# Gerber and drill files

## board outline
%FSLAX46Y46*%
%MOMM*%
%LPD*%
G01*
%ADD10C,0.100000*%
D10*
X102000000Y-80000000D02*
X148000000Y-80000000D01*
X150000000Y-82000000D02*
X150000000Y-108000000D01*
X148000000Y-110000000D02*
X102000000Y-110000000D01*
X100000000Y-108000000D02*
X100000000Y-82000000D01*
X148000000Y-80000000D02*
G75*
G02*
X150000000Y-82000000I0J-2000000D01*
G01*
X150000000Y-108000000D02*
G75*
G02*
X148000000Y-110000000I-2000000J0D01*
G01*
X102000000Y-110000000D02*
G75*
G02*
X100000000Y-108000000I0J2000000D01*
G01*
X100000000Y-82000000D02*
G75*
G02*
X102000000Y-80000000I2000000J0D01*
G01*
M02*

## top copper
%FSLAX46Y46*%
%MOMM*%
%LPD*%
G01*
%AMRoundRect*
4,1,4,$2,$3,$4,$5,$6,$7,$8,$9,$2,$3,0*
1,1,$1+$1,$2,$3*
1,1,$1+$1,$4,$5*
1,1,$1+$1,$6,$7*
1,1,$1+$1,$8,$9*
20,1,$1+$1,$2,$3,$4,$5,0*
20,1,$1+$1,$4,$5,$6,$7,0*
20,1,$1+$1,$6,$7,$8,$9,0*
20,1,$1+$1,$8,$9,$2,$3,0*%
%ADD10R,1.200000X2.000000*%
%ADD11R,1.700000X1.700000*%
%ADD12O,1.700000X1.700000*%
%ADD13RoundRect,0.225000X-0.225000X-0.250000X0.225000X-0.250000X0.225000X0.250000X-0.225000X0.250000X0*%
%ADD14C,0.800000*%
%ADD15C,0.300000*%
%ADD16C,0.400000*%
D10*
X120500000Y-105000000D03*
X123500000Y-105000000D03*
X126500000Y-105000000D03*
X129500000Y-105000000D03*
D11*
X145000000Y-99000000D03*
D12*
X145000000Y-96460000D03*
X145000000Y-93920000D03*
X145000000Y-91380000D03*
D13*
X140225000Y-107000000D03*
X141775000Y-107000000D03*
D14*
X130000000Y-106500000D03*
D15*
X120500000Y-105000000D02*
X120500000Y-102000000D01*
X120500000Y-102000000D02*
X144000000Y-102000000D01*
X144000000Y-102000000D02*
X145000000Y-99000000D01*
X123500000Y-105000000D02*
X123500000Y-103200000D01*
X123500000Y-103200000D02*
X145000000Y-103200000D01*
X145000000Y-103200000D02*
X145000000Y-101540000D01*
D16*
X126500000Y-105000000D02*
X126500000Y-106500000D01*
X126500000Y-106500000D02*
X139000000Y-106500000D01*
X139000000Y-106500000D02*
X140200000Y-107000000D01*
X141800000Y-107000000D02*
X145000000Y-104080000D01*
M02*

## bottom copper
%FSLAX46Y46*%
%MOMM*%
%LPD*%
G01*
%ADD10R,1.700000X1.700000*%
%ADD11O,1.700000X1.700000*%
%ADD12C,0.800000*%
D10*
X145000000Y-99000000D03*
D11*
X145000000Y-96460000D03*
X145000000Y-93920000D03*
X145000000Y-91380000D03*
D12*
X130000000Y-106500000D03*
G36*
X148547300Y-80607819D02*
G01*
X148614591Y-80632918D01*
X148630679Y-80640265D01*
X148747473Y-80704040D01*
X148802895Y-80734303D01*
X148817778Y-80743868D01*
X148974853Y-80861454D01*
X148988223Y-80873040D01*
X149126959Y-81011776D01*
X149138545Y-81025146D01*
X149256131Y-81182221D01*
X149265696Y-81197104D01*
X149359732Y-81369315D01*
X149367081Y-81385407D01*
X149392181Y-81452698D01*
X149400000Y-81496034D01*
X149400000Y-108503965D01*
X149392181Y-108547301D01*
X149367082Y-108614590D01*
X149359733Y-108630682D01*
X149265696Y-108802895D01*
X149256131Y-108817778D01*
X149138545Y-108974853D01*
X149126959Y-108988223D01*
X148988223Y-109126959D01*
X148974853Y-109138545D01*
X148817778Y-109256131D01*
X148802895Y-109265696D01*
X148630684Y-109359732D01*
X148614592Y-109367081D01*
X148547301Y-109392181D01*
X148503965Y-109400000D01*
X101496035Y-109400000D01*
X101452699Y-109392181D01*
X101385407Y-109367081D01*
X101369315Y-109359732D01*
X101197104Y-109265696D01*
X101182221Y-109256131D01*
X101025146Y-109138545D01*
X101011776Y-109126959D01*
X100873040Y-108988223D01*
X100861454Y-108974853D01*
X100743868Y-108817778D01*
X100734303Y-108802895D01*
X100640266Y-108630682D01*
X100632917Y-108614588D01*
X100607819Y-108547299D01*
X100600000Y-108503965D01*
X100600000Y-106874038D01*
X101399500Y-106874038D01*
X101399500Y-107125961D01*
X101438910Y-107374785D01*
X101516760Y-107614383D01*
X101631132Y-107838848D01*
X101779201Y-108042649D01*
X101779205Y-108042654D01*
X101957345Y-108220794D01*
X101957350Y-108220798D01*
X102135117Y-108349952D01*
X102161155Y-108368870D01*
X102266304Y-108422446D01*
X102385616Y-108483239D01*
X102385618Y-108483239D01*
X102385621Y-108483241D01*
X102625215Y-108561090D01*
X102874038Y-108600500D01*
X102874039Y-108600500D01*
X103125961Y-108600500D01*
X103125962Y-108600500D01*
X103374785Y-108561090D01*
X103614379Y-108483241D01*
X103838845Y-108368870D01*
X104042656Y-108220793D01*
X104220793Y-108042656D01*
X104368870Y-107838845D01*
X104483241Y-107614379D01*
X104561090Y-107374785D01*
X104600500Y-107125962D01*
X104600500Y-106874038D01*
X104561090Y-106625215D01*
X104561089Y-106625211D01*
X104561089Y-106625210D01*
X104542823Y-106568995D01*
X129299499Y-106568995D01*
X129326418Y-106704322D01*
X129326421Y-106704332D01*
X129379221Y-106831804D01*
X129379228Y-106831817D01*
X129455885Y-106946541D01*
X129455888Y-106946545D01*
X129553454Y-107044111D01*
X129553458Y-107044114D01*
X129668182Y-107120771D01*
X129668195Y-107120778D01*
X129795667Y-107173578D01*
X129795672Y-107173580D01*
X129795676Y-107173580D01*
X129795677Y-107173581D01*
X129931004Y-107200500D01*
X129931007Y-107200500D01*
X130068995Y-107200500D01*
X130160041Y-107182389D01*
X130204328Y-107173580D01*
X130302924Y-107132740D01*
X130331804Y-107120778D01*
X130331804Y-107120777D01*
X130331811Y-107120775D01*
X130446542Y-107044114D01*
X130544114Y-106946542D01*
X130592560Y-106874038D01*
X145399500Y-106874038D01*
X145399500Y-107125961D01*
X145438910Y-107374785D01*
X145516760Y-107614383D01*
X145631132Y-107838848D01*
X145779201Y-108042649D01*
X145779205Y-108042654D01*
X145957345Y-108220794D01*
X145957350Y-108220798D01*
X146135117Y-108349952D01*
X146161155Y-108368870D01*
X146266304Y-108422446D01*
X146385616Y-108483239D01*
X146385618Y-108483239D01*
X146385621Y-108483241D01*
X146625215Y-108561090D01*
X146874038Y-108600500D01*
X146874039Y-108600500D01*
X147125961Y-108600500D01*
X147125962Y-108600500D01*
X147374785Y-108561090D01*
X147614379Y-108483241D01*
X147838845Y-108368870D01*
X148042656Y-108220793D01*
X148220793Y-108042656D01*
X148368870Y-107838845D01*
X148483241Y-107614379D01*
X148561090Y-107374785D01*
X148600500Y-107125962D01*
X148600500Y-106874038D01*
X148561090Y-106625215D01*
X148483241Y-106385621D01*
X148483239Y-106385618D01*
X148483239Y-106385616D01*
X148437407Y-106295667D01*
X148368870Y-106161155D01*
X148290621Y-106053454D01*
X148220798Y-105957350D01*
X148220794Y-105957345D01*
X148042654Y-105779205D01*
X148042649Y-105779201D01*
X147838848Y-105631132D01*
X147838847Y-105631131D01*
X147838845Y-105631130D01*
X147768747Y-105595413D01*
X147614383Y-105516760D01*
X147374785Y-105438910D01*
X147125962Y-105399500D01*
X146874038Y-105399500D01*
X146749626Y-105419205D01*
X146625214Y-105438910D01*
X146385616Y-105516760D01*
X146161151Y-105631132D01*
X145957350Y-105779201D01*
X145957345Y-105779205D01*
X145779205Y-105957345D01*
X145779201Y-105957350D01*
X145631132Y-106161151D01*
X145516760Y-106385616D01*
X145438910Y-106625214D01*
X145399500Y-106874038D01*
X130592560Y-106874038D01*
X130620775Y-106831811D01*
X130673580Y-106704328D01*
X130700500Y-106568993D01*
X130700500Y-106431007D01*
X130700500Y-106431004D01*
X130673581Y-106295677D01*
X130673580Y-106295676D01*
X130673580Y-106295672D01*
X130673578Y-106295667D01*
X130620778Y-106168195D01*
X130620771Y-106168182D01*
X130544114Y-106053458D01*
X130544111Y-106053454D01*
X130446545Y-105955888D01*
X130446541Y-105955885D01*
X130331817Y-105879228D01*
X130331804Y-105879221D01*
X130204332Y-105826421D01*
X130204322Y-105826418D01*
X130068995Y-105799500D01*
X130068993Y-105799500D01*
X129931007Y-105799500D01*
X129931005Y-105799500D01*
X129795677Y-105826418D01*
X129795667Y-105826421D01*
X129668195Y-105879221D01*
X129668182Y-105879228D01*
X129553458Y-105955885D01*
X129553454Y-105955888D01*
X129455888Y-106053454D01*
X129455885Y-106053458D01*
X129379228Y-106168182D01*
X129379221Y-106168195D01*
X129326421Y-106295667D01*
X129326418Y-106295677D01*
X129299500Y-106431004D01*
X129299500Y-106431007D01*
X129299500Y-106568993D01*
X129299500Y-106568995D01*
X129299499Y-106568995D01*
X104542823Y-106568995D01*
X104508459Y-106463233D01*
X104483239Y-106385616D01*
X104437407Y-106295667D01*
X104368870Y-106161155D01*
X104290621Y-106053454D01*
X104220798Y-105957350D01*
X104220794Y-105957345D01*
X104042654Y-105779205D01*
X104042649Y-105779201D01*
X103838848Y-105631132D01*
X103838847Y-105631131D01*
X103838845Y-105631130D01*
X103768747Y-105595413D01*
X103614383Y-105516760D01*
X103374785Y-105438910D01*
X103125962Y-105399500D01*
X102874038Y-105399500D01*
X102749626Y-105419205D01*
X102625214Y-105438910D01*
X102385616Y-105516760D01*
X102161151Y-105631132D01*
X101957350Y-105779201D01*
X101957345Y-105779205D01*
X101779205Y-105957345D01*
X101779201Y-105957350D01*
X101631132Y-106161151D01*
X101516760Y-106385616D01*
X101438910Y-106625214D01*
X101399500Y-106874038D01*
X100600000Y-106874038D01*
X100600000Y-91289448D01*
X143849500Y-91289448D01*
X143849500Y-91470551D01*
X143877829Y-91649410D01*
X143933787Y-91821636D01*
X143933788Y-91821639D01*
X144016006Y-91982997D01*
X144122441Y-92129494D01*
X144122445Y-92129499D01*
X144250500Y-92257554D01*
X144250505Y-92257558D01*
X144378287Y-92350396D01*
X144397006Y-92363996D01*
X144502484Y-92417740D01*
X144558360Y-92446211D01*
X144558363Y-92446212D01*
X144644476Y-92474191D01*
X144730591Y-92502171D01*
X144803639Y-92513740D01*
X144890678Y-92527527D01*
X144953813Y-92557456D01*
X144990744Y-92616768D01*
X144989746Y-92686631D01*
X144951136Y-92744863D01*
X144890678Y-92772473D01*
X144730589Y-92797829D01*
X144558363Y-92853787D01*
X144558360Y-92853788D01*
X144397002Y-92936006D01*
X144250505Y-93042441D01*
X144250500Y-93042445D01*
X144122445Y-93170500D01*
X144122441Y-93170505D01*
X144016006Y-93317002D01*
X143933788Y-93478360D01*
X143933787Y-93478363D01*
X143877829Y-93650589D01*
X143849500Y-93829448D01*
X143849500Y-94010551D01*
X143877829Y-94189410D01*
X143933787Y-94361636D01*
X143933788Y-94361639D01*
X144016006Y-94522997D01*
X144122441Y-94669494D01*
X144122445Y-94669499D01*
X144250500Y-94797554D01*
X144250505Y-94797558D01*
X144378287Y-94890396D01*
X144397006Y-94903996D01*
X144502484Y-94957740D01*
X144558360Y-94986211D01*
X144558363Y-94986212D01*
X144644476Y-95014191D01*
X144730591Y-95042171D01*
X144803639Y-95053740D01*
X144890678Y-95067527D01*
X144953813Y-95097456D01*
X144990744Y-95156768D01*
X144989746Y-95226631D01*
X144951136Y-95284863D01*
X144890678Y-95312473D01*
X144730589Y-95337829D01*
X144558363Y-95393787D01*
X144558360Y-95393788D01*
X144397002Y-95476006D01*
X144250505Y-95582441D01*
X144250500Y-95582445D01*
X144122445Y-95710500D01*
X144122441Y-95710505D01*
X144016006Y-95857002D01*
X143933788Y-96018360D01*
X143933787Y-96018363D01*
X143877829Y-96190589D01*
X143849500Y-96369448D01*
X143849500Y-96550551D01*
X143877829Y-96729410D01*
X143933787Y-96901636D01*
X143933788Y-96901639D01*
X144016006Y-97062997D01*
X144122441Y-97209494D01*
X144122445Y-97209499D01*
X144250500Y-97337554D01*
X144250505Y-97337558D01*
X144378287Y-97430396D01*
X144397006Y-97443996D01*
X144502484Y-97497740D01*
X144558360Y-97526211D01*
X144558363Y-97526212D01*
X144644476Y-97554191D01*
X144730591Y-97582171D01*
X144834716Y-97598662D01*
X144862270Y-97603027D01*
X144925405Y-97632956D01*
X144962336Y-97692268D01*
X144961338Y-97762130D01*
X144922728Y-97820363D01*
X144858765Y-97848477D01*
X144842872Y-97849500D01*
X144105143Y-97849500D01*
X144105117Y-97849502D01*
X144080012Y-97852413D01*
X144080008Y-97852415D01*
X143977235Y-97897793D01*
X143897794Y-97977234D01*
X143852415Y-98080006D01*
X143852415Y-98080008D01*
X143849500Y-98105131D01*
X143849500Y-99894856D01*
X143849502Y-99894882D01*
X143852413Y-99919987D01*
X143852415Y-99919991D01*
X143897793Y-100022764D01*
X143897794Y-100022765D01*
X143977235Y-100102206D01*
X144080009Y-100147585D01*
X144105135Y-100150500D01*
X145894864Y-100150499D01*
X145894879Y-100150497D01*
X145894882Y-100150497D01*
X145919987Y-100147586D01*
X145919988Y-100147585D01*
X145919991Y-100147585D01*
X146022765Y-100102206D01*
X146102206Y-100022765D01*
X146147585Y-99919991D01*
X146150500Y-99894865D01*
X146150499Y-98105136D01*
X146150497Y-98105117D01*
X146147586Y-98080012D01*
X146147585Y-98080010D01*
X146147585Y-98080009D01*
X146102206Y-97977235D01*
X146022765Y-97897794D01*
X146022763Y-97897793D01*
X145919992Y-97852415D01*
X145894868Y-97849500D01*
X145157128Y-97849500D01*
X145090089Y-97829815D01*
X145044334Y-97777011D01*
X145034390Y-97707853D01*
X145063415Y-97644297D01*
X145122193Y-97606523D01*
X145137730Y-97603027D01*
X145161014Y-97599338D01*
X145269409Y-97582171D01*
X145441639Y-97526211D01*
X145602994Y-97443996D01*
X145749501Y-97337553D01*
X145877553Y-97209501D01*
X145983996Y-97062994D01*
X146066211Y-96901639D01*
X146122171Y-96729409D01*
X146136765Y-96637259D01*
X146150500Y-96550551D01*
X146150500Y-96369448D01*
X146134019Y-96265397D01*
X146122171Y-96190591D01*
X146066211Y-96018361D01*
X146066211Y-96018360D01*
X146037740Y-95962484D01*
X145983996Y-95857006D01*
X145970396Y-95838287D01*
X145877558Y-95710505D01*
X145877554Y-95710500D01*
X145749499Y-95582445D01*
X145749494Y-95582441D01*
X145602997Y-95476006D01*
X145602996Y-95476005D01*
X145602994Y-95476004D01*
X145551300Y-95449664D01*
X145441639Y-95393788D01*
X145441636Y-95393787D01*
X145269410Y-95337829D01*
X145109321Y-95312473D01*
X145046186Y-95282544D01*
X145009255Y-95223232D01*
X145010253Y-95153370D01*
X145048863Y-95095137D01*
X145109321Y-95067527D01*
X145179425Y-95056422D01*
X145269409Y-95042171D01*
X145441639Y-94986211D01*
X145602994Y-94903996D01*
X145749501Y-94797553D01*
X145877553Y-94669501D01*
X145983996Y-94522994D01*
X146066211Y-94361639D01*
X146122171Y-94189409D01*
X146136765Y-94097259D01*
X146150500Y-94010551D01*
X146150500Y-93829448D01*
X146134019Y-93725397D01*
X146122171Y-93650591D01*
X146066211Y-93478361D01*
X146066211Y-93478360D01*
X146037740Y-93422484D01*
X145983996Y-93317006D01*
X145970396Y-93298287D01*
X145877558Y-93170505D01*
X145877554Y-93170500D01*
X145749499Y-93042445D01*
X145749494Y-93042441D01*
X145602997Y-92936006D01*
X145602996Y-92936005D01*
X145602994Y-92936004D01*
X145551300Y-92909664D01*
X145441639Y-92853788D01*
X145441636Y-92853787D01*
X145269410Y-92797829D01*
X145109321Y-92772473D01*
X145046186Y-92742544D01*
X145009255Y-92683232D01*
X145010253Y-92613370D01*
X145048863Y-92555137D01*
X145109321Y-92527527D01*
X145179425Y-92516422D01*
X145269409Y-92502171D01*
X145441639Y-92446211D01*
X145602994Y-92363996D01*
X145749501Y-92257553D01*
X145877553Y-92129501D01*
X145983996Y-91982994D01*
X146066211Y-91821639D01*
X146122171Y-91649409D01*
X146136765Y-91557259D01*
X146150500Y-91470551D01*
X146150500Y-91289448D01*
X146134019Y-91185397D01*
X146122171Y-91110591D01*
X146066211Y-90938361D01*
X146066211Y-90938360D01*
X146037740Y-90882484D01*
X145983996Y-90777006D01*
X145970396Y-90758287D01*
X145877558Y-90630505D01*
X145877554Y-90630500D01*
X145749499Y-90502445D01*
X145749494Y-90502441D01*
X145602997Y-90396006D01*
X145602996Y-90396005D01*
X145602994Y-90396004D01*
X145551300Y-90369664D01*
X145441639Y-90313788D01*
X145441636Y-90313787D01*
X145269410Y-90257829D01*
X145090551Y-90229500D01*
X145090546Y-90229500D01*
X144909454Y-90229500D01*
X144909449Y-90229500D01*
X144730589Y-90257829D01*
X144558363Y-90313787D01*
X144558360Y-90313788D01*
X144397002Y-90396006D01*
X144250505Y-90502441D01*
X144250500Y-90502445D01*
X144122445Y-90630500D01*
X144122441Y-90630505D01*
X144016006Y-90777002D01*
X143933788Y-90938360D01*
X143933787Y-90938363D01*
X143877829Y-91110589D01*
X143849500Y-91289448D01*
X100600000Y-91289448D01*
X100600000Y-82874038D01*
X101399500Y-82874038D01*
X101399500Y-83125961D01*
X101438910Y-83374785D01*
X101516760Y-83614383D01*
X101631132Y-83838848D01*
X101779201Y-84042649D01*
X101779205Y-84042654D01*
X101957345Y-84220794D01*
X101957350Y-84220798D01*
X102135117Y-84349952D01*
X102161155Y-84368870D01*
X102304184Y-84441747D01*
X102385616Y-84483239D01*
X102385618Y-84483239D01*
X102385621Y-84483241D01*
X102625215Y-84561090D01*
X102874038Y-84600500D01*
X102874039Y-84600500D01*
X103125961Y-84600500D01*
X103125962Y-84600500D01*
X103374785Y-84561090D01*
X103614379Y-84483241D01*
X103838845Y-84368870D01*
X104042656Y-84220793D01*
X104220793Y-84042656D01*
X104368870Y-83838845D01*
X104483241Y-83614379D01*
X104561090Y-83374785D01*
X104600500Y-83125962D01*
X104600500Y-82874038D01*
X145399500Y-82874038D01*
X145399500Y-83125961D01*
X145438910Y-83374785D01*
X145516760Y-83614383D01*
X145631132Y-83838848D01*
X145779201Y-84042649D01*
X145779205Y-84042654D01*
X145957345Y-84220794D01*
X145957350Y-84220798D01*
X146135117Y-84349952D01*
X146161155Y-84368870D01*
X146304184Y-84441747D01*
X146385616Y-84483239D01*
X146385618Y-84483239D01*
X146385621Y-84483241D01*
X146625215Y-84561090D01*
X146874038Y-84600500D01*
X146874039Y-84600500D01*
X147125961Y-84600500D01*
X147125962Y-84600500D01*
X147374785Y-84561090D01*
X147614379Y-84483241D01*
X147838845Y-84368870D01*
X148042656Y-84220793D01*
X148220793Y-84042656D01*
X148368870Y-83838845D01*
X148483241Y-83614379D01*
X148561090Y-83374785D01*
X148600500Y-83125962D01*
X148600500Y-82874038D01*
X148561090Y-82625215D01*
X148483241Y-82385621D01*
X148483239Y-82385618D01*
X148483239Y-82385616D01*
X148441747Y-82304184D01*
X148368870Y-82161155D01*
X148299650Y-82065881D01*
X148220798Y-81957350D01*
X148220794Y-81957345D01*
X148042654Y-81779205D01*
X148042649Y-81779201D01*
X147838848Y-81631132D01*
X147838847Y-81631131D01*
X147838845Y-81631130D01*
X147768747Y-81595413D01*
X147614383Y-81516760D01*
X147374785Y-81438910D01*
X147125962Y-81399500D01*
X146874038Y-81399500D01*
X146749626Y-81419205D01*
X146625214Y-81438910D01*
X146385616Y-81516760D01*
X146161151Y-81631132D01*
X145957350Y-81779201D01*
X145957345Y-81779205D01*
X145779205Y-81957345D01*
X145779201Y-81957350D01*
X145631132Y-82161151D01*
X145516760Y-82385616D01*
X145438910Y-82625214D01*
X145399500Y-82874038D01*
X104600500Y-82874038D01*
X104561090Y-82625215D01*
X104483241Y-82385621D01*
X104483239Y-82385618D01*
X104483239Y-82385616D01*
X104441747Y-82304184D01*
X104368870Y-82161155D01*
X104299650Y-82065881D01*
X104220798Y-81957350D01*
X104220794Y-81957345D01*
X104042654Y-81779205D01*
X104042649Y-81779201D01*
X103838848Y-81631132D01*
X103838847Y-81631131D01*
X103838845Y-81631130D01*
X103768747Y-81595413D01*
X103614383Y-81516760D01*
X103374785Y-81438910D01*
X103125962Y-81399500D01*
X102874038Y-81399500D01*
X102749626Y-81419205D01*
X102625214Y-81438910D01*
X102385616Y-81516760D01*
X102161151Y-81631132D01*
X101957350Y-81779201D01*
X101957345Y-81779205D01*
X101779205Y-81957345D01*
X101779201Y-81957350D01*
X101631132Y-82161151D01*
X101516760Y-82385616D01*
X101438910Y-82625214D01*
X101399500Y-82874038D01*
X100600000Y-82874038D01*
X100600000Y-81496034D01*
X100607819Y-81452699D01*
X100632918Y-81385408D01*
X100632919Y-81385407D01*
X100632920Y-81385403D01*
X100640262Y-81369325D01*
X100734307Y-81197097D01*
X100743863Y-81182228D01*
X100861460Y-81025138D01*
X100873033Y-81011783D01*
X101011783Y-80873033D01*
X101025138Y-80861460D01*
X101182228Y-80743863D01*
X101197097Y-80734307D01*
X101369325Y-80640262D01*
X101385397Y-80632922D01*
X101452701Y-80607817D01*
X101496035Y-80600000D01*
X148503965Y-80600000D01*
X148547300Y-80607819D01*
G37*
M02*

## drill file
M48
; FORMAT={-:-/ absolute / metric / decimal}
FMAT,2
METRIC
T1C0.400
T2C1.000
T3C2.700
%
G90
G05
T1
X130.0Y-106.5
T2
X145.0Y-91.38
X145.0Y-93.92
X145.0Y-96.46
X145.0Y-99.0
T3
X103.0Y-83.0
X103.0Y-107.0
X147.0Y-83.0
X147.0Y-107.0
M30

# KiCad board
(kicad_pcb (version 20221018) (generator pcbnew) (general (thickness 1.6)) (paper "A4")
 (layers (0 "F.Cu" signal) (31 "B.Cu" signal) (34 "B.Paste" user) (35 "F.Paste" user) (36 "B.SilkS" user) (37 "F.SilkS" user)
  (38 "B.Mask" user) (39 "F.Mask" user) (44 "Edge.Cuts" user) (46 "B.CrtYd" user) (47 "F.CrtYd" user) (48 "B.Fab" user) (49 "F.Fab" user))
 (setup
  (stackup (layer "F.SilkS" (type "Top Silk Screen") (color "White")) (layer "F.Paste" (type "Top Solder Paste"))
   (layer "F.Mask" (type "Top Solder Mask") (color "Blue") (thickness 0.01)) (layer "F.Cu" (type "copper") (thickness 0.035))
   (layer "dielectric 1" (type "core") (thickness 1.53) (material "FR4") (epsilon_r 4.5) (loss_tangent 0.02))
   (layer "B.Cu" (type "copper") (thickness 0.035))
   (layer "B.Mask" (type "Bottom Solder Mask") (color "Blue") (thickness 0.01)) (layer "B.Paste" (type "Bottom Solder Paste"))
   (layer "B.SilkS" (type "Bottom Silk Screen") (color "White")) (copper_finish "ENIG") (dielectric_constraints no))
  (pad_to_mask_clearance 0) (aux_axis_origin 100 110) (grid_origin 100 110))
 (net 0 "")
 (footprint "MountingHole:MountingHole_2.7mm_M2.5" (layer "F.Cu") (at 103 83) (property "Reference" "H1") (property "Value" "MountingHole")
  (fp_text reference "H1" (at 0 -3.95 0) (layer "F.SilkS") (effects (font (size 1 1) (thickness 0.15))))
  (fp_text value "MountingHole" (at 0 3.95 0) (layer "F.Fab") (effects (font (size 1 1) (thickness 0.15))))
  (pad "" np_thru_hole circle (at 0 0) (size 2.7 2.7) (drill 2.7) (layers "*.Cu" "*.Mask")))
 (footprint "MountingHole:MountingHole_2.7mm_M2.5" (layer "F.Cu") (at 147 83) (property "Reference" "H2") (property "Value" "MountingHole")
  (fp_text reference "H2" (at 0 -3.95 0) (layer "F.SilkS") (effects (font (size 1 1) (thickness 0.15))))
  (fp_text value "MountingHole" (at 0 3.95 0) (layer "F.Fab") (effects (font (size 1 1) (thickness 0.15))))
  (pad "" np_thru_hole circle (at 0 0) (size 2.7 2.7) (drill 2.7) (layers "*.Cu" "*.Mask")))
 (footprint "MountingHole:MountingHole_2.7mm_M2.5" (layer "F.Cu") (at 103 107) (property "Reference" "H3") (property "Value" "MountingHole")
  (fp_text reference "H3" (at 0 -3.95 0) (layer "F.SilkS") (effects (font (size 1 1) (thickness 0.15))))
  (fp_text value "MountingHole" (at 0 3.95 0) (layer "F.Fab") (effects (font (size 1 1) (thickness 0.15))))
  (pad "" np_thru_hole circle (at 0 0) (size 2.7 2.7) (drill 2.7) (layers "*.Cu" "*.Mask")))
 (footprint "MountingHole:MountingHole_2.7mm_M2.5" (layer "F.Cu") (at 147 107) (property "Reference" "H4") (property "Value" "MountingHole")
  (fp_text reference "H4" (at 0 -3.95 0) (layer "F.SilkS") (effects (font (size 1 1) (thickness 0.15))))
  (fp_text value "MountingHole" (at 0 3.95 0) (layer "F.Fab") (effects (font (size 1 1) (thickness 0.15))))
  (pad "" np_thru_hole circle (at 0 0) (size 2.7 2.7) (drill 2.7) (layers "*.Cu" "*.Mask")))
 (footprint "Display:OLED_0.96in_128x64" (layer "F.Cu") (at 125 94) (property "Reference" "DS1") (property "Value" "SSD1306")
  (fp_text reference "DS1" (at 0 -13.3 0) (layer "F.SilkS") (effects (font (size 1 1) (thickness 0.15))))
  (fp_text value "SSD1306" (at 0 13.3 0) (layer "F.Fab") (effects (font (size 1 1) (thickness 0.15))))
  (pad "1" smd rect (at -4.5 11) (size 1.2 2) (layers "F.Cu" "F.Paste" "F.Mask"))
  (pad "2" smd rect (at -1.5 11) (size 1.2 2) (layers "F.Cu" "F.Paste" "F.Mask"))
  (pad "3" smd rect (at 1.5 11) (size 1.2 2) (layers "F.Cu" "F.Paste" "F.Mask"))
  (pad "4" smd rect (at 4.5 11) (size 1.2 2) (layers "F.Cu" "F.Paste" "F.Mask")))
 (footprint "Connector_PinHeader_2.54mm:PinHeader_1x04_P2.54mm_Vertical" (layer "B.Cu") (at 145 99) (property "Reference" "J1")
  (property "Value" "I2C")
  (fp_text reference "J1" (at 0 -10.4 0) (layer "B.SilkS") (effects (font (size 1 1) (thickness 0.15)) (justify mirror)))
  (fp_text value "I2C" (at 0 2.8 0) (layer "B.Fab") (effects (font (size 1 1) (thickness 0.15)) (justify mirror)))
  (pad "1" thru_hole rect (at 0 0) (size 1.7 1.7) (drill 1) (layers "*.Cu" "*.Mask"))
  (pad "2" thru_hole oval (at 0 -2.54) (size 1.7 1.7) (drill 1) (layers "*.Cu" "*.Mask"))
  (pad "3" thru_hole oval (at 0 -5.08) (size 1.7 1.7) (drill 1) (layers "*.Cu" "*.Mask"))
  (pad "4" thru_hole oval (at 0 -7.62) (size 1.7 1.7) (drill 1) (layers "*.Cu" "*.Mask")))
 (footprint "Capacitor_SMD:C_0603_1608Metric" (layer "F.Cu") (at 141 107) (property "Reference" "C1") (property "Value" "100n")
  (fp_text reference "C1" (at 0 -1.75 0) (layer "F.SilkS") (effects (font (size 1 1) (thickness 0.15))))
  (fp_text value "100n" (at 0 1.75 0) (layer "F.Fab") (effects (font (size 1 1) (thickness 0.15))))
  (pad "1" smd roundrect (at -0.775 0) (size 0.9 0.95) (layers "F.Cu" "F.Paste" "F.Mask"))
  (pad "2" smd roundrect (at 0.775 0) (size 0.9 0.95) (layers "F.Cu" "F.Paste" "F.Mask")))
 (gr_line (start 102 80) (end 148 80) (stroke (width 0.1) (type solid)) (layer "Edge.Cuts"))
 (gr_line (start 150 82) (end 150 108) (stroke (width 0.1) (type solid)) (layer "Edge.Cuts"))
 (gr_line (start 148 110) (end 102 110) (stroke (width 0.1) (type solid)) (layer "Edge.Cuts"))
 (gr_line (start 100 108) (end 100 82) (stroke (width 0.1) (type solid)) (layer "Edge.Cuts"))
 (gr_arc (start 148 80) (mid 149.4142 80.5858) (end 150 82) (stroke (width 0.1) (type solid)) (layer "Edge.Cuts"))
 (gr_arc (start 150 108) (mid 149.4142 109.4142) (end 148 110) (stroke (width 0.1) (type solid)) (layer "Edge.Cuts"))
 (gr_arc (start 102 110) (mid 100.5858 109.4142) (end 100 108) (stroke (width 0.1) (type solid)) (layer "Edge.Cuts"))
 (gr_arc (start 100 82) (mid 100.5858 80.5858) (end 102 80) (stroke (width 0.1) (type solid)) (layer "Edge.Cuts"))
 (segment (start 120.5 105) (end 120.5 102) (width 0.3) (layer "F.Cu") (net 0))
 (segment (start 120.5 102) (end 144 102) (width 0.3) (layer "F.Cu") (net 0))
 (segment (start 144 102) (end 145 99) (width 0.3) (layer "F.Cu") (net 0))
 (segment (start 123.5 105) (end 123.5 103.2) (width 0.3) (layer "F.Cu") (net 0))
 (segment (start 123.5 103.2) (end 145 103.2) (width 0.3) (layer "F.Cu") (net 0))
 (segment (start 145 103.2) (end 145 101.54) (width 0.3) (layer "F.Cu") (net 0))
 (segment (start 126.5 105) (end 126.5 106.5) (width 0.4) (layer "F.Cu") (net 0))
 (segment (start 126.5 106.5) (end 139 106.5) (width 0.4) (layer "F.Cu") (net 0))
 (segment (start 139 106.5) (end 140.2 107) (width 0.4) (layer "F.Cu") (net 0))
 (segment (start 141.8 107) (end 145 104.08) (width 0.4) (layer "F.Cu") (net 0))
 (via (at 130 106.5) (size 0.8) (drill 0.4) (layers "F.Cu" "B.Cu") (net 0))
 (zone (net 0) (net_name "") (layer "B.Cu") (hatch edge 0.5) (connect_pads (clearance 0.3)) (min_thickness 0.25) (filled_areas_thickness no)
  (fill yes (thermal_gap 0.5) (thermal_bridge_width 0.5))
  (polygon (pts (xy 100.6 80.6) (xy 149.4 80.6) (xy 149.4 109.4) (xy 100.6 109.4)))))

